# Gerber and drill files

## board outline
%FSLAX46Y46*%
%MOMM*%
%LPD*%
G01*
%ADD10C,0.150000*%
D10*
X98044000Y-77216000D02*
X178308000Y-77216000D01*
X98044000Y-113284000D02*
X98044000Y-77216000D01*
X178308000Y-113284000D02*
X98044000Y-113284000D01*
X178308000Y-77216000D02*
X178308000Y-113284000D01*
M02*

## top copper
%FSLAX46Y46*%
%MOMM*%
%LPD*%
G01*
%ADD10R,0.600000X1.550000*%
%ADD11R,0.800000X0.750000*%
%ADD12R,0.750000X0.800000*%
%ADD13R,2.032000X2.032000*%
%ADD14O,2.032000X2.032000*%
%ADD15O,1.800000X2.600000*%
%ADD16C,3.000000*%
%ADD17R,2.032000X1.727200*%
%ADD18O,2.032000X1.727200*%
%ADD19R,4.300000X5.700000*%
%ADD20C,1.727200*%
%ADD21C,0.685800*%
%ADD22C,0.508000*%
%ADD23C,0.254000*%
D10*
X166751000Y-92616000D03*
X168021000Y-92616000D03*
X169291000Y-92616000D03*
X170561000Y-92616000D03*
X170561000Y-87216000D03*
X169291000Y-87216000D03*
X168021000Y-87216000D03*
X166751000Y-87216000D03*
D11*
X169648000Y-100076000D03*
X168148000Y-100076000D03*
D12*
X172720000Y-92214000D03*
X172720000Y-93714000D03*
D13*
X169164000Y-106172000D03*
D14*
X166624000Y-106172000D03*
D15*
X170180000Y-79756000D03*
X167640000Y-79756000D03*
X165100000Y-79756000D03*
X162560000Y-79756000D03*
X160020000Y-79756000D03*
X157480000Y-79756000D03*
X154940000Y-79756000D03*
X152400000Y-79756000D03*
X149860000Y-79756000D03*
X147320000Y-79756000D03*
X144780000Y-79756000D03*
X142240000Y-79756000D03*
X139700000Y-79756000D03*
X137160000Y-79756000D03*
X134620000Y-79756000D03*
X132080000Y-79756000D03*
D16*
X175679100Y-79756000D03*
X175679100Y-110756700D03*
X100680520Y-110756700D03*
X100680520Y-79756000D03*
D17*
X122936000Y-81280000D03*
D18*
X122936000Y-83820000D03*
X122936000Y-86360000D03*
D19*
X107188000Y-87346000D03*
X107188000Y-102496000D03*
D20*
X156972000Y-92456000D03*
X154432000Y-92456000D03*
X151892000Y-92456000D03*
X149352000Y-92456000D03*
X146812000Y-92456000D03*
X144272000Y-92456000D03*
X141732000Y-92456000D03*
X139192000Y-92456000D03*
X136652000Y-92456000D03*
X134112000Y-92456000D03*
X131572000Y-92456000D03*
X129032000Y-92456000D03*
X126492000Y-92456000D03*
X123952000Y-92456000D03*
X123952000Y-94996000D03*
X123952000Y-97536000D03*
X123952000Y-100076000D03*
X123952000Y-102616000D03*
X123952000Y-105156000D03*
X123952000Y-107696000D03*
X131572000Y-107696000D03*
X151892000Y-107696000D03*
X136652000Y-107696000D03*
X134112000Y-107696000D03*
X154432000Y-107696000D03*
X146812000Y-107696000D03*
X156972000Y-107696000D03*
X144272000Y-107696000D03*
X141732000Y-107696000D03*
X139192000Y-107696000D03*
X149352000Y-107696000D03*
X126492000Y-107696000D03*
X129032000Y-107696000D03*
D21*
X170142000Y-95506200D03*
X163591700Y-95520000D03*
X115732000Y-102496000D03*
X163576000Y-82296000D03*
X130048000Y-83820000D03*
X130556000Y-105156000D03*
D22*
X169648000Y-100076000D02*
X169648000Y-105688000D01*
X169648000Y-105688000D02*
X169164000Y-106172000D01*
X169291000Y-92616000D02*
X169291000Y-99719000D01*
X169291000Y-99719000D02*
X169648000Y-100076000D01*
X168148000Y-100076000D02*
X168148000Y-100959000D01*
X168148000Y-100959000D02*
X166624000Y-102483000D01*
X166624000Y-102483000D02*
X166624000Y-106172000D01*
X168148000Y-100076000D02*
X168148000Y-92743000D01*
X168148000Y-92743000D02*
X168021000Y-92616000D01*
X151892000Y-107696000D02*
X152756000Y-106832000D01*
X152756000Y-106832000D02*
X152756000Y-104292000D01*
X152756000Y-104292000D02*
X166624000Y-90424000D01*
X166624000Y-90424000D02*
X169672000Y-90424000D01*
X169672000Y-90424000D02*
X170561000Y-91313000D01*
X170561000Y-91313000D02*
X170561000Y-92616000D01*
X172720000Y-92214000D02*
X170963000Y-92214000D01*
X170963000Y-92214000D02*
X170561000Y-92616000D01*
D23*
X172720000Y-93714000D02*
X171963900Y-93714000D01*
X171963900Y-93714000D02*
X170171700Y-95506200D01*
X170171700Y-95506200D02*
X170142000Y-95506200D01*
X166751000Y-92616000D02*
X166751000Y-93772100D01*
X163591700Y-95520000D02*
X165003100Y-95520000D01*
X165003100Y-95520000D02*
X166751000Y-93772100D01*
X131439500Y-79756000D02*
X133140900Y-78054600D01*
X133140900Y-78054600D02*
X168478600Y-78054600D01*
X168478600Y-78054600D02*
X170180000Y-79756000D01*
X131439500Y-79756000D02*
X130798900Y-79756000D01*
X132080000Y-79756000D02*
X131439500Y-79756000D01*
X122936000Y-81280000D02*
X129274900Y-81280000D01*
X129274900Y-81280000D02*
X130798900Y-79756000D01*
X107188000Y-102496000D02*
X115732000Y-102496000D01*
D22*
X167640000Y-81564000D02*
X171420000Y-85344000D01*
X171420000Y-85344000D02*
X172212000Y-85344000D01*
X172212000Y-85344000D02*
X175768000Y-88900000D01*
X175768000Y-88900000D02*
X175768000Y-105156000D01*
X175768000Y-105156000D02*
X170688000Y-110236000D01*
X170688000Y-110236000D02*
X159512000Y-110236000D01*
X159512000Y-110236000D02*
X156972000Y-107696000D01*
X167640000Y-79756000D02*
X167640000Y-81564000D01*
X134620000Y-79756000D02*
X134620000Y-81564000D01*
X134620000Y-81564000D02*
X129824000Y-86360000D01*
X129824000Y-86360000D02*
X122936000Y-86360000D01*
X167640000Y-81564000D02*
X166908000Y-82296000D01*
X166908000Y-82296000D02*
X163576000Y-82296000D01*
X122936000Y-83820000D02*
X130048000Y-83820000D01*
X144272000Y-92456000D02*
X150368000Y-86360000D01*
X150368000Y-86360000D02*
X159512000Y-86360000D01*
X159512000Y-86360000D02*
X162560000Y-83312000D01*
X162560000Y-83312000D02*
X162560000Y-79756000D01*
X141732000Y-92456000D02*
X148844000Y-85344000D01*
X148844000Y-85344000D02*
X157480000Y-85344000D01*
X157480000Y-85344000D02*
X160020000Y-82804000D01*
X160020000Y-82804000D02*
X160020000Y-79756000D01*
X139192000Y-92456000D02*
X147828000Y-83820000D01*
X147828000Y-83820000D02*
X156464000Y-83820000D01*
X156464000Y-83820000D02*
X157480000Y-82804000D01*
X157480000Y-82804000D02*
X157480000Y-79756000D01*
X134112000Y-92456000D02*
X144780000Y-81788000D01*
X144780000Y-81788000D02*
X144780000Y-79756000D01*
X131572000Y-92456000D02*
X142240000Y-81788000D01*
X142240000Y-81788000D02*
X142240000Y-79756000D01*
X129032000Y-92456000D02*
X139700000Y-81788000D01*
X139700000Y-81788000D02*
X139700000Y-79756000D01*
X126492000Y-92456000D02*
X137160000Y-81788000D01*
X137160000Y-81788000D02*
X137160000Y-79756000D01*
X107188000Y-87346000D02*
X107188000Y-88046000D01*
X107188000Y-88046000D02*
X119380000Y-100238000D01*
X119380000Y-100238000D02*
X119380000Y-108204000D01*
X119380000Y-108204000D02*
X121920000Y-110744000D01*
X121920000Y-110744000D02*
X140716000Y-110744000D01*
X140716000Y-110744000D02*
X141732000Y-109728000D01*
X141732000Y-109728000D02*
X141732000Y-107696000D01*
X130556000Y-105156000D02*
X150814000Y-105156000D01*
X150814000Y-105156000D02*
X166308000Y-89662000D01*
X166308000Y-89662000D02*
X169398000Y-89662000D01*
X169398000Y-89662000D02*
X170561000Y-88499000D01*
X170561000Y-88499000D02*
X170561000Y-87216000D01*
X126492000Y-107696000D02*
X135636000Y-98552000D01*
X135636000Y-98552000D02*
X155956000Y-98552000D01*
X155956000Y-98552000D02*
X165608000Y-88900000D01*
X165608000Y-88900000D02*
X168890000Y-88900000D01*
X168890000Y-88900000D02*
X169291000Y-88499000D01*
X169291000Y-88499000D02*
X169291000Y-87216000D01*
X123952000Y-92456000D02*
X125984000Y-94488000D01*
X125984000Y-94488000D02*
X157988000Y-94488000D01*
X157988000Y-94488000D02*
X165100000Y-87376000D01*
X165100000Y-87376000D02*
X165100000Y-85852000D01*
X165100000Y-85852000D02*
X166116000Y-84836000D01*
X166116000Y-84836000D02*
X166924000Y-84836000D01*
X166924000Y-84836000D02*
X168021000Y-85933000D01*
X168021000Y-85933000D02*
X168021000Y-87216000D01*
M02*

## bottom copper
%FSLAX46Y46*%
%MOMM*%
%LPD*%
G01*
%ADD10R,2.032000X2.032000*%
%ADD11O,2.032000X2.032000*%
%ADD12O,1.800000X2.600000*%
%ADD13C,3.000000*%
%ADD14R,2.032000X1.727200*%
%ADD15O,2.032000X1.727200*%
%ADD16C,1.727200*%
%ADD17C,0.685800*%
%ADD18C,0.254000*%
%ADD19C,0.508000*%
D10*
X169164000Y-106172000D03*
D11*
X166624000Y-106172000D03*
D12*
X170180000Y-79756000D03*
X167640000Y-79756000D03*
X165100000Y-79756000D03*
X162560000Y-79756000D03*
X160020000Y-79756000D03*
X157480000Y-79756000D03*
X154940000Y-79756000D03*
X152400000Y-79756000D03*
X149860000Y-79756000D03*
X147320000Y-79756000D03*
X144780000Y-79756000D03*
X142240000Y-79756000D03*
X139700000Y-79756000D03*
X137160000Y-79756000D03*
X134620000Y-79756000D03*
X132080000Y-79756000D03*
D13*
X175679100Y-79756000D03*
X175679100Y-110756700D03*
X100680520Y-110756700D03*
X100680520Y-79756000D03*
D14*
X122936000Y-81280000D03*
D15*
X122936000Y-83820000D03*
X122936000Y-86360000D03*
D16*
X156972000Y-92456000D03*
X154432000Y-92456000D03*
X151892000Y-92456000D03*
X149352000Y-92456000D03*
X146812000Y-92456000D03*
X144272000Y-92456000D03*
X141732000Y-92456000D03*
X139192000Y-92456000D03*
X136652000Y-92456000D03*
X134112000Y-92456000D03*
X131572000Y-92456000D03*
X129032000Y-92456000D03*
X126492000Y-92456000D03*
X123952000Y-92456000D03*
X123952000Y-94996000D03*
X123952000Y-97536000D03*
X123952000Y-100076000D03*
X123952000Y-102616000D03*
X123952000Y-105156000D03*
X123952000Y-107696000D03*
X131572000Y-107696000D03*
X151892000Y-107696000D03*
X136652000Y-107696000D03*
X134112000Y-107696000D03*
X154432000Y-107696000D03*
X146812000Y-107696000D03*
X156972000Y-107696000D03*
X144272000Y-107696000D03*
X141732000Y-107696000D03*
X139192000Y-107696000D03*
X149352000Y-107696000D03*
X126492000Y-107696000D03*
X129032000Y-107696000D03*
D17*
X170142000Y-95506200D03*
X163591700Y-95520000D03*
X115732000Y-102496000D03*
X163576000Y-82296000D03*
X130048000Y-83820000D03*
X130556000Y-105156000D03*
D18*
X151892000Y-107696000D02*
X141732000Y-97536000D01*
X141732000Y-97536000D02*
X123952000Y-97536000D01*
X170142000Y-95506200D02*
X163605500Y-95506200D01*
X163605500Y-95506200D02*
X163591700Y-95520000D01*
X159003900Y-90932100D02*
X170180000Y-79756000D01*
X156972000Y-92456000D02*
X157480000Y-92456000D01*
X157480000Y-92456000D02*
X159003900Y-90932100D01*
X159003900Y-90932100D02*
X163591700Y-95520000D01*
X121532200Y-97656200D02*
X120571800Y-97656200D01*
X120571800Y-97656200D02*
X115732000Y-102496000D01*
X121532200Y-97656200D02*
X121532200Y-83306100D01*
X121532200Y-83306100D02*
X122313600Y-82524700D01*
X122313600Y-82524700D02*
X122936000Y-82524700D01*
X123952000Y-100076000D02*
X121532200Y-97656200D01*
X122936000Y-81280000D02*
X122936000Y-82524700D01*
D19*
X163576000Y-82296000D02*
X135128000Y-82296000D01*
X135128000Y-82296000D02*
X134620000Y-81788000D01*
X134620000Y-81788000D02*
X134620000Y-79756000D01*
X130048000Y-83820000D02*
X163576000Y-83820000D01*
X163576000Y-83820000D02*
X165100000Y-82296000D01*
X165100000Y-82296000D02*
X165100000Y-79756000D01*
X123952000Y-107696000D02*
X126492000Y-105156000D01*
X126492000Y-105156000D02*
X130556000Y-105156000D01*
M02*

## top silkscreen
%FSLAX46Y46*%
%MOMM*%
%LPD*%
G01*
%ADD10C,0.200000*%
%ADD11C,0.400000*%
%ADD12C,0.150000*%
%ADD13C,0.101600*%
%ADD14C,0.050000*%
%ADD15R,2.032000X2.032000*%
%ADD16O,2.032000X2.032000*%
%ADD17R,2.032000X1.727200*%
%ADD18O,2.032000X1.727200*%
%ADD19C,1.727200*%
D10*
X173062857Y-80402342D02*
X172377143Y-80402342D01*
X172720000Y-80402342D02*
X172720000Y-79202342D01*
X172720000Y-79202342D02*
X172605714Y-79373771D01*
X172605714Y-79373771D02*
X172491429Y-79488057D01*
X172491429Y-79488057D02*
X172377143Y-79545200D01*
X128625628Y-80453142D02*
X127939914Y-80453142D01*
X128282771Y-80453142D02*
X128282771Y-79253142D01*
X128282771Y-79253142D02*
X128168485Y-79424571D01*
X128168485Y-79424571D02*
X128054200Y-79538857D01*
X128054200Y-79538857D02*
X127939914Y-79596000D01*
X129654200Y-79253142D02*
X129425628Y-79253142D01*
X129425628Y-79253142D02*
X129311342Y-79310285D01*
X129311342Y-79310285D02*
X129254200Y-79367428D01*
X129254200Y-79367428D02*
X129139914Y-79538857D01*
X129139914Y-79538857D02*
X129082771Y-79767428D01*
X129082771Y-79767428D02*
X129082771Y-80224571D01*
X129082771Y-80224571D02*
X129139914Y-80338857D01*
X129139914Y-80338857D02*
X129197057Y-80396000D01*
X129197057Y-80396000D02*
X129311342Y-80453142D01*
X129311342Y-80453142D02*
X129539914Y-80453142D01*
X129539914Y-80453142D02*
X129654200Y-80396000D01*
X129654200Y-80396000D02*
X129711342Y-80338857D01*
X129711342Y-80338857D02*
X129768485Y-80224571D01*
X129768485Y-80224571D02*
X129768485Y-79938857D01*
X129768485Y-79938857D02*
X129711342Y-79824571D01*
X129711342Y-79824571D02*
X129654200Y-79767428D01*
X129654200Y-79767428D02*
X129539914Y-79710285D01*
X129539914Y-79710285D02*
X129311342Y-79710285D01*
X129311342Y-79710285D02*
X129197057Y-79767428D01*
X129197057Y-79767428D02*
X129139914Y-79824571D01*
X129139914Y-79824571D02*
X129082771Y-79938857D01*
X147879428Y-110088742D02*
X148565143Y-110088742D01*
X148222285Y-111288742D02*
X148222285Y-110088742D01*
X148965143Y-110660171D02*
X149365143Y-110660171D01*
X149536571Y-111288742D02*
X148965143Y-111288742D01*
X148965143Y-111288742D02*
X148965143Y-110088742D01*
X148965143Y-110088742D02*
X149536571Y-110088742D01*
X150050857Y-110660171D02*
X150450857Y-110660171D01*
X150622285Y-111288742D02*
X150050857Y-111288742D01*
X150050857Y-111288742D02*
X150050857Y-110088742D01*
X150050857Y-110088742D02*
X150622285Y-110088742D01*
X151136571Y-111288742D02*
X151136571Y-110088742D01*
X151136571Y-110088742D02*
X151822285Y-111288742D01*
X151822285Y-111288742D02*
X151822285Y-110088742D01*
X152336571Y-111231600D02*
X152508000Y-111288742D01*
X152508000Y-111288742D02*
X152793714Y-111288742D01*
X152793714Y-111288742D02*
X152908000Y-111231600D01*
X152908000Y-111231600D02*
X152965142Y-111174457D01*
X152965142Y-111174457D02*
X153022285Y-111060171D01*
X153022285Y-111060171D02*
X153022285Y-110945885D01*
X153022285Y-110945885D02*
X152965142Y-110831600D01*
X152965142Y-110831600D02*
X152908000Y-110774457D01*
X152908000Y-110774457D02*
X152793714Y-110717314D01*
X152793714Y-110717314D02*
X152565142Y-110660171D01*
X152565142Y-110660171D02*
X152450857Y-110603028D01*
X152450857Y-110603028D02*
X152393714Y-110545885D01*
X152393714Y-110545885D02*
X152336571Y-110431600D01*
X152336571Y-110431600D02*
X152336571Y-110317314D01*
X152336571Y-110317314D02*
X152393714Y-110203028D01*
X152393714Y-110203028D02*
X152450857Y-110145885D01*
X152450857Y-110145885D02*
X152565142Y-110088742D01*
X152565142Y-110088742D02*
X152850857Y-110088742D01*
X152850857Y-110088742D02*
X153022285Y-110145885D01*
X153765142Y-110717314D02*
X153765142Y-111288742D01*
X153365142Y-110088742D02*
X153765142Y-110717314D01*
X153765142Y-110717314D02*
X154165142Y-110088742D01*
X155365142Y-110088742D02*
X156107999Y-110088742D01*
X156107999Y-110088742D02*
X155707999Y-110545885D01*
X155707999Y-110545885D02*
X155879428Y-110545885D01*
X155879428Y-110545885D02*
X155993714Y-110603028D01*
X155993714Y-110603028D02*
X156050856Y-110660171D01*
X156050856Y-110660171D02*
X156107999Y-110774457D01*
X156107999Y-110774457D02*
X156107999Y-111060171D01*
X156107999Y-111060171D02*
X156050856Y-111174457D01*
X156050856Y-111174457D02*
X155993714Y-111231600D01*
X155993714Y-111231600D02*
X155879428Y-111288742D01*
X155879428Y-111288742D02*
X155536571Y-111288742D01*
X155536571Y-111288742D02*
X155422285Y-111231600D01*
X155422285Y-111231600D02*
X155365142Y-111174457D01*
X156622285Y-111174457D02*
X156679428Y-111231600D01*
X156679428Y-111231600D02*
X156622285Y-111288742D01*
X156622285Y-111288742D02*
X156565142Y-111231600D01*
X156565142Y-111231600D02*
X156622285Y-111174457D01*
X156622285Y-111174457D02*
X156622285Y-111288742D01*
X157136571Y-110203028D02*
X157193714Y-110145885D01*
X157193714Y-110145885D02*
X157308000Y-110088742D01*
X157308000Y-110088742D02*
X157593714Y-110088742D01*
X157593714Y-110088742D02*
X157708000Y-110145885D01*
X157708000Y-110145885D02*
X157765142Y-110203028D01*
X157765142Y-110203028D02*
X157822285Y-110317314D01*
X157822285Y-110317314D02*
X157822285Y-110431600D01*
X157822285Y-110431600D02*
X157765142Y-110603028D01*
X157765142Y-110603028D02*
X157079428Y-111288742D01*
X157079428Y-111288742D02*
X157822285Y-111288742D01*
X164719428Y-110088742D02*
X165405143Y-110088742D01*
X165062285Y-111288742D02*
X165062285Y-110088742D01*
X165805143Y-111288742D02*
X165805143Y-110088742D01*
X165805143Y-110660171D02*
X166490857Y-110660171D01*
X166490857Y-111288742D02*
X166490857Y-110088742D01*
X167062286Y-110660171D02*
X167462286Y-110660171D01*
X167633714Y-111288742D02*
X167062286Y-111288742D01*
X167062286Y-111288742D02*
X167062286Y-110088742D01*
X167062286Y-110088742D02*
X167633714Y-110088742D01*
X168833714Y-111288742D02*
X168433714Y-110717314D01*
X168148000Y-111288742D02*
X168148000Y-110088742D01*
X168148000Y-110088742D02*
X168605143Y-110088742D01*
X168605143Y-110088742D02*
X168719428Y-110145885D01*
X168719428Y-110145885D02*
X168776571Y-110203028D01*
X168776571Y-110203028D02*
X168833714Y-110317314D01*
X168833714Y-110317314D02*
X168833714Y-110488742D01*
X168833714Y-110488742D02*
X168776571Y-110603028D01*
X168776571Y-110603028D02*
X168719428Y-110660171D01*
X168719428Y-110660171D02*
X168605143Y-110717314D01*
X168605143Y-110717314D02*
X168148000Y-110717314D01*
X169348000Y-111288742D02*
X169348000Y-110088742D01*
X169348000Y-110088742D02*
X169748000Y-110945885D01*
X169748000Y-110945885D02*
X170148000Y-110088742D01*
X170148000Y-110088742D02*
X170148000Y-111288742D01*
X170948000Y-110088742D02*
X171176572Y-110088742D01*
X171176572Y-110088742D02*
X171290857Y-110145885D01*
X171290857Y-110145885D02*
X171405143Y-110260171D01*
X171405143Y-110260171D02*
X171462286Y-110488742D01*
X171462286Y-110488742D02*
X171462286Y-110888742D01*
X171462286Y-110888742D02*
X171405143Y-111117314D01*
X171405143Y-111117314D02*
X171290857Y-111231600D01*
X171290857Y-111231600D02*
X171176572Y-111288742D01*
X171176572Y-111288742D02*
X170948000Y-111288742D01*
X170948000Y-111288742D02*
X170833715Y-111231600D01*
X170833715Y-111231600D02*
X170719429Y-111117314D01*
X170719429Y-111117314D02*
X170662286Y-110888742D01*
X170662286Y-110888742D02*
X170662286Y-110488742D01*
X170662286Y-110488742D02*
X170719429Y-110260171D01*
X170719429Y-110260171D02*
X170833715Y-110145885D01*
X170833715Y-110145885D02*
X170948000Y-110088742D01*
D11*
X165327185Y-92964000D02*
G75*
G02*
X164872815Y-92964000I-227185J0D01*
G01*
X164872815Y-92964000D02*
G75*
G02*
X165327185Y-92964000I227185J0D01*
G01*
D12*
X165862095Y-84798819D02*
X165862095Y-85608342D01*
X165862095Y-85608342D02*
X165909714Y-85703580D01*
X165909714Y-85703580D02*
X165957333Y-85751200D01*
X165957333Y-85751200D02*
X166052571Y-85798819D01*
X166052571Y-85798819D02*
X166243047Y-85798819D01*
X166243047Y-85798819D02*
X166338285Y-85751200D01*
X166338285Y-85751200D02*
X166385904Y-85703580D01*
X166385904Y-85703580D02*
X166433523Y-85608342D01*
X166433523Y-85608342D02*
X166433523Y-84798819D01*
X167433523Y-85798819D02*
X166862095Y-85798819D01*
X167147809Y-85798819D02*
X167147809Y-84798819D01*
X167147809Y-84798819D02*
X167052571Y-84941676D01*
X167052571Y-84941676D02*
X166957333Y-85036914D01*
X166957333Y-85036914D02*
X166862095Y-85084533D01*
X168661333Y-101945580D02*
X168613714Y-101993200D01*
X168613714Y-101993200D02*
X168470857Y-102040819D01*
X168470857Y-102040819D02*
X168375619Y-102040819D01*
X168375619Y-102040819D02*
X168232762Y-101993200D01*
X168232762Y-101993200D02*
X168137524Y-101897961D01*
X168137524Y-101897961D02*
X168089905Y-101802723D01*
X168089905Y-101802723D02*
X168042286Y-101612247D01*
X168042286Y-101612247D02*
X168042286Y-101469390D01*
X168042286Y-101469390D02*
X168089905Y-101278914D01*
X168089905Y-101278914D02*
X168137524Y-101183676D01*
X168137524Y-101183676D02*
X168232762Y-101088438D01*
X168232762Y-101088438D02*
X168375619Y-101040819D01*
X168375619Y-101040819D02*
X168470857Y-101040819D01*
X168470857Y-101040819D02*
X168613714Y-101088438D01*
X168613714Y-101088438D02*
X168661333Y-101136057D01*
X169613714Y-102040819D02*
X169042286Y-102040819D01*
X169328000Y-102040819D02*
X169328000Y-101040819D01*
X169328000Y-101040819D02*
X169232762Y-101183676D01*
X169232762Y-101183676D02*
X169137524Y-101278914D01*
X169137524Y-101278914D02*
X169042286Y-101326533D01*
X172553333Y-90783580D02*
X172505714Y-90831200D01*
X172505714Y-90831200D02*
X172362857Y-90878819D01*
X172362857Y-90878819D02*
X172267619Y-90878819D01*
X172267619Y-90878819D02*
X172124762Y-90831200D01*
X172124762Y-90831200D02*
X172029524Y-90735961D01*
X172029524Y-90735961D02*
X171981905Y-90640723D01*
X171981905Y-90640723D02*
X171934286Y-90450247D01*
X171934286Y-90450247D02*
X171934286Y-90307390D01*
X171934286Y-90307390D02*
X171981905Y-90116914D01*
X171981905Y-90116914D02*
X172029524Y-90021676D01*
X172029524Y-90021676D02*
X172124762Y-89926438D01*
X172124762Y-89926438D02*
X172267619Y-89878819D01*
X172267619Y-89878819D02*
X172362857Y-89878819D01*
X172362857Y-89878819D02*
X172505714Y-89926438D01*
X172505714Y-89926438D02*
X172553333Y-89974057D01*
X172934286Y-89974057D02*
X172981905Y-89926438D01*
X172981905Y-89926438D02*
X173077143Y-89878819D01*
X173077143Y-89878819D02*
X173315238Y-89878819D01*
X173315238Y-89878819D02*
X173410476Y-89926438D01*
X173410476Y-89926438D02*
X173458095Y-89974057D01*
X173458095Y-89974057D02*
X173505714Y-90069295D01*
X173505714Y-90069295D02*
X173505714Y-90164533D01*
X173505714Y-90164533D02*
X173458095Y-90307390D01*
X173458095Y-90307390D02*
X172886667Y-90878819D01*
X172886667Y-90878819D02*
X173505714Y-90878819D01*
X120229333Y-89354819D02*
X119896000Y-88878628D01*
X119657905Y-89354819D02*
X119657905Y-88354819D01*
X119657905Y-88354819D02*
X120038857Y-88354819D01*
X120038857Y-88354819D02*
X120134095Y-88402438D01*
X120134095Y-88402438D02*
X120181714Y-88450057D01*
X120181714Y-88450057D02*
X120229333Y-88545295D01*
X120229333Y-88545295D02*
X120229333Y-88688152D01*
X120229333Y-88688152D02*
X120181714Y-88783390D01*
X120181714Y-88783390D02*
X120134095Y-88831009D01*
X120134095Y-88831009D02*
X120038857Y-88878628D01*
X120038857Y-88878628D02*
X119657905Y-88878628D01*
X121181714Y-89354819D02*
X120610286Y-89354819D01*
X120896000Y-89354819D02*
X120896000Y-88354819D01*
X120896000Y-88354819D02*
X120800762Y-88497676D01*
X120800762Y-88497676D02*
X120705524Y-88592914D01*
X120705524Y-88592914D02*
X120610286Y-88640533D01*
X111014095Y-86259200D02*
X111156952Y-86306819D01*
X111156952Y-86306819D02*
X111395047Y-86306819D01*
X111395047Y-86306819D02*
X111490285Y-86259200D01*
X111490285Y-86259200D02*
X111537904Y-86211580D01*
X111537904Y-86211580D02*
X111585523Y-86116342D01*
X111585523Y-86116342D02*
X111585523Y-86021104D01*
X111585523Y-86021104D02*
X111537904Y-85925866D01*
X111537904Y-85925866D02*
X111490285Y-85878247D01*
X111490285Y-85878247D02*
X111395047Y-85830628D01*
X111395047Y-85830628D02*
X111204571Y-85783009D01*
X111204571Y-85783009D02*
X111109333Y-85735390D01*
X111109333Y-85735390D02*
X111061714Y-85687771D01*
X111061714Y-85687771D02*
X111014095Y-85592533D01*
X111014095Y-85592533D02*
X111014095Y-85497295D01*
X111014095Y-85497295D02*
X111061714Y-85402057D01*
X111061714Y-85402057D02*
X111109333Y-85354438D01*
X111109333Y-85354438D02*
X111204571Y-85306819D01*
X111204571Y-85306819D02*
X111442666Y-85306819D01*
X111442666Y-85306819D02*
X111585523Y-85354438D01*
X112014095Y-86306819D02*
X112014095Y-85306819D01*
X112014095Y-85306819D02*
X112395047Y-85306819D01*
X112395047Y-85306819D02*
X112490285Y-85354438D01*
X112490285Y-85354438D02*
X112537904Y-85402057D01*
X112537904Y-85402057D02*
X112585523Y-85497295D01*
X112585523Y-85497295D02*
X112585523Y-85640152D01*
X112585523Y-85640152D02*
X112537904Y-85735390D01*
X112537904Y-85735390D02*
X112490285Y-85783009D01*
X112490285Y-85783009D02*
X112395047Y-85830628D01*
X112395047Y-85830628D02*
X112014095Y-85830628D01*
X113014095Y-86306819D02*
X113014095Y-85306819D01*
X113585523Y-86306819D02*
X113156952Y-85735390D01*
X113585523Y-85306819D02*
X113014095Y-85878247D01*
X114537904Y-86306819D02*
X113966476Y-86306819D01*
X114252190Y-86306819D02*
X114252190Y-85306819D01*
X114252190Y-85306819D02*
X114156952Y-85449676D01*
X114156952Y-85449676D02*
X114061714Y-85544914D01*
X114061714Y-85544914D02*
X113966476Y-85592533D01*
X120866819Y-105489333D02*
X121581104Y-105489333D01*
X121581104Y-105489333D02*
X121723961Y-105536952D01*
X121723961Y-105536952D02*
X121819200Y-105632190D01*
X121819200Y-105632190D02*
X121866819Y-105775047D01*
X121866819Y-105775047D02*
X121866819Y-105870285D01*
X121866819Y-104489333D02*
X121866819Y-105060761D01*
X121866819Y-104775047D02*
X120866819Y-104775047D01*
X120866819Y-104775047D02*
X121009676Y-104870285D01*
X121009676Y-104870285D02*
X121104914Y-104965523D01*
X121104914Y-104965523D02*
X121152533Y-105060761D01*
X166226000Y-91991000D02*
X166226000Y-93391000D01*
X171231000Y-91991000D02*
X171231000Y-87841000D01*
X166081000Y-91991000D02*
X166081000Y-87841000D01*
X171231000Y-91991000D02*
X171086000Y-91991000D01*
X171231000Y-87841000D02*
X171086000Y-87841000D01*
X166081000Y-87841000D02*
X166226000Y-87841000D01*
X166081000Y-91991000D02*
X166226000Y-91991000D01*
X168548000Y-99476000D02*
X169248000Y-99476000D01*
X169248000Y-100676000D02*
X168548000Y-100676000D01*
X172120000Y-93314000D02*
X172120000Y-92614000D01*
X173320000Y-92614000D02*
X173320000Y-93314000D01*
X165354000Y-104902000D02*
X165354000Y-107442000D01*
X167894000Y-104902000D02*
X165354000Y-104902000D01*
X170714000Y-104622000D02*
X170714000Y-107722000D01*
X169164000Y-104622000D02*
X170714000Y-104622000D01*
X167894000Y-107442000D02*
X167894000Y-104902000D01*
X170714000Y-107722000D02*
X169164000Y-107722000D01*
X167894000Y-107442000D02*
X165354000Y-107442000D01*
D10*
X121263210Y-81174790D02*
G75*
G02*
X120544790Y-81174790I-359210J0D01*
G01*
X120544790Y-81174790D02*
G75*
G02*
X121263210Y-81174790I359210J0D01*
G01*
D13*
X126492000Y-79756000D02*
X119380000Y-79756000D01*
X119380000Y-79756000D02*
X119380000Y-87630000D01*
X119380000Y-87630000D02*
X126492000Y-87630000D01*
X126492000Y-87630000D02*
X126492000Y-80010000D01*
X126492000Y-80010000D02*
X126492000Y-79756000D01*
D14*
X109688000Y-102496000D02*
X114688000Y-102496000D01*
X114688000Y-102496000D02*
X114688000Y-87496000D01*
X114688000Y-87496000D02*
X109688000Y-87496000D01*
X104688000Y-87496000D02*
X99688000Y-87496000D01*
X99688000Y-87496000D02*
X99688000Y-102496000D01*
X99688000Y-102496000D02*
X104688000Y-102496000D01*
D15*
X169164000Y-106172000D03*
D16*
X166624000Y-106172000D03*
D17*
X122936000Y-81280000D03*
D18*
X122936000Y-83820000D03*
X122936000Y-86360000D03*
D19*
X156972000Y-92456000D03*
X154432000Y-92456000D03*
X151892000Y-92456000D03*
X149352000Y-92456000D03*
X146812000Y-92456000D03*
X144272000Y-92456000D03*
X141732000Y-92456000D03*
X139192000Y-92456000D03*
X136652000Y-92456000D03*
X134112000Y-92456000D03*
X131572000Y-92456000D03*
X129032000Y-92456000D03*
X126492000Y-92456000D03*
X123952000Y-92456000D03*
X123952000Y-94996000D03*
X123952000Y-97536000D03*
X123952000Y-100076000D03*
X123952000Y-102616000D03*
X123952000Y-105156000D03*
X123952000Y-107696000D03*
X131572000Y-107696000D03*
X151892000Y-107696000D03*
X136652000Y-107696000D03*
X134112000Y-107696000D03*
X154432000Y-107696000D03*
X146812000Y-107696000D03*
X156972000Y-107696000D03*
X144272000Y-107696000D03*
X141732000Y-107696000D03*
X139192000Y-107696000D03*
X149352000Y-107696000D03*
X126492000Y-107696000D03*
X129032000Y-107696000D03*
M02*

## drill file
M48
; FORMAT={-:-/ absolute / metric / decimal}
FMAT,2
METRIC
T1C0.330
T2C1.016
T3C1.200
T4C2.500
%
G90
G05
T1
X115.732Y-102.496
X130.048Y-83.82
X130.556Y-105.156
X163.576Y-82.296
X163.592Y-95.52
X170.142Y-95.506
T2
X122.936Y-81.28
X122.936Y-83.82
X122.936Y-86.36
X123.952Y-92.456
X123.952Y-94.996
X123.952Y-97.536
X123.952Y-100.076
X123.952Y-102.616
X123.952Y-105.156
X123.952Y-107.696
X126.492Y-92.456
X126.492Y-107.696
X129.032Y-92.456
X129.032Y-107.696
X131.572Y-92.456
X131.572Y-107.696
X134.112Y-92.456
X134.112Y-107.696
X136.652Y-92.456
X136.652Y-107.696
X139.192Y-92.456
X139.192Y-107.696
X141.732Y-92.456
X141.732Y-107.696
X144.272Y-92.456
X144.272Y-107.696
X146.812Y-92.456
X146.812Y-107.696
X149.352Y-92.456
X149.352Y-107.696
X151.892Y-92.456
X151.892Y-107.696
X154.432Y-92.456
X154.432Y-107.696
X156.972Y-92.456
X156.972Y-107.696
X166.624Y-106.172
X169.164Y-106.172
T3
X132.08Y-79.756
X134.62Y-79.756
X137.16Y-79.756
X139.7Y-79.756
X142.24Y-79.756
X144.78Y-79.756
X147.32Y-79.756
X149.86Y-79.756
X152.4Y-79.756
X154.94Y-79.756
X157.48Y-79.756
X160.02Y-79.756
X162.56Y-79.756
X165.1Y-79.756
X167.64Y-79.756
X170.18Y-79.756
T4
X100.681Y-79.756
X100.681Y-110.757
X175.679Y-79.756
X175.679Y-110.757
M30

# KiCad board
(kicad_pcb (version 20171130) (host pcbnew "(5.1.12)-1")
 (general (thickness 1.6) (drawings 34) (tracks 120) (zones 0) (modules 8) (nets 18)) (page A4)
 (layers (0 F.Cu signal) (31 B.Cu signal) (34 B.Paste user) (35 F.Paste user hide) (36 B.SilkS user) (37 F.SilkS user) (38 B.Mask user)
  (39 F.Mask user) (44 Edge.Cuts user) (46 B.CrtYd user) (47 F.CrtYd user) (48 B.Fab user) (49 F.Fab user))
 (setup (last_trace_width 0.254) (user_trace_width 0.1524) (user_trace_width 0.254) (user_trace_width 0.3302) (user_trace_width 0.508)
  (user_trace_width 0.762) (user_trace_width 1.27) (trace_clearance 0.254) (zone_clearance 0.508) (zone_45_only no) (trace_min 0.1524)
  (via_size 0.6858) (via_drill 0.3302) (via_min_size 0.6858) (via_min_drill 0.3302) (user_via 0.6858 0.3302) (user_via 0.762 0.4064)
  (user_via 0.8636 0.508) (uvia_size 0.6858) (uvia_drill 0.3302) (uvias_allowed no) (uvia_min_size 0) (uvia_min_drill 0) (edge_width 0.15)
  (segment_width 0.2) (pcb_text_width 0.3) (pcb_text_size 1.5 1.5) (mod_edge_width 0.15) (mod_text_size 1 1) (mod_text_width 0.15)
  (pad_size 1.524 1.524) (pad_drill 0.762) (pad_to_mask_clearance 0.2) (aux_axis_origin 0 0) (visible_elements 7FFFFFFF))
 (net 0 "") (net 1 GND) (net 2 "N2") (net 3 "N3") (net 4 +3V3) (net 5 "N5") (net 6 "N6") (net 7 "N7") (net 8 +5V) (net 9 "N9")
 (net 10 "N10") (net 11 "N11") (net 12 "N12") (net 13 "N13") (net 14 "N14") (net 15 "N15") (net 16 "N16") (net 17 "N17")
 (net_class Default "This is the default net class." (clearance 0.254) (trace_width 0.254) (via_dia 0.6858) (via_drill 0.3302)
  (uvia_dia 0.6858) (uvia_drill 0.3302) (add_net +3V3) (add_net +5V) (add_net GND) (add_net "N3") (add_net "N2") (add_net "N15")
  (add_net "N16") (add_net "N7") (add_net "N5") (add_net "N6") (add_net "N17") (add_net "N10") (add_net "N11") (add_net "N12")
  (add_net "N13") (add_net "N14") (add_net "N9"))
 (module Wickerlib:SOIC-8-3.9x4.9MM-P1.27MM (layer F.Cu) (at 168.656 89.916 90)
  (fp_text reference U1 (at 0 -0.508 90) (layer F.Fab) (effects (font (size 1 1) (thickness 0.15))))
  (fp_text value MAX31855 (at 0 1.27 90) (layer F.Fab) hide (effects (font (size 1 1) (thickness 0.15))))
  (fp_line (start -2.075 -2.43) (end -3.475 -2.43) (layer F.SilkS) (width 0.15))
  (fp_line (start -2.075 2.575) (end 2.075 2.575) (layer F.SilkS) (width 0.15))
  (fp_line (start -2.075 -2.575) (end 2.075 -2.575) (layer F.SilkS) (width 0.15))
  (fp_line (start -2.075 2.575) (end -2.075 2.43) (layer F.SilkS) (width 0.15))
  (fp_line (start 2.075 2.575) (end 2.075 2.43) (layer F.SilkS) (width 0.15))
  (fp_line (start 2.075 -2.575) (end 2.075 -2.43) (layer F.SilkS) (width 0.15))
  (fp_line (start -2.075 -2.575) (end -2.075 -2.43) (layer F.SilkS) (width 0.15))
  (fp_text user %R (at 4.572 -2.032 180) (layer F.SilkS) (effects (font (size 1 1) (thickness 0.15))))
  (pad 1 smd rect (at -2.7 -1.905 90) (size 1.55 0.6) (layers F.Cu F.Paste F.Mask) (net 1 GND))
  (pad 2 smd rect (at -2.7 -0.635 90) (size 1.55 0.6) (layers F.Cu F.Paste F.Mask) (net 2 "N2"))
  (pad 3 smd rect (at -2.7 0.635 90) (size 1.55 0.6) (layers F.Cu F.Paste F.Mask) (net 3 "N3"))
  (pad 4 smd rect (at -2.7 1.905 90) (size 1.55 0.6) (layers F.Cu F.Paste F.Mask) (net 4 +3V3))
  (pad 5 smd rect (at 2.7 1.905 90) (size 1.55 0.6) (layers F.Cu F.Paste F.Mask) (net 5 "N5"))
  (pad 6 smd rect (at 2.7 0.635 90) (size 1.55 0.6) (layers F.Cu F.Paste F.Mask) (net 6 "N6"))
  (pad 7 smd rect (at 2.7 -0.635 90) (size 1.55 0.6) (layers F.Cu F.Paste F.Mask) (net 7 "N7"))
  (pad 8 smd rect (at 2.7 -1.905 90) (size 1.55 0.6) (layers F.Cu F.Paste F.Mask)))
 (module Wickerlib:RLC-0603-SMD (layer F.Cu) (at 168.898 100.076 180)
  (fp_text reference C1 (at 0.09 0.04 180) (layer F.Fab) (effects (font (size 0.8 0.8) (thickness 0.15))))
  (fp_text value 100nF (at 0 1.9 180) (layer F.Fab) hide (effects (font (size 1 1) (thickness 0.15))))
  (fp_line (start 0.35 0.6) (end -0.35 0.6) (layer F.SilkS) (width 0.15))
  (fp_line (start -0.35 -0.6) (end 0.35 -0.6) (layer F.SilkS) (width 0.15))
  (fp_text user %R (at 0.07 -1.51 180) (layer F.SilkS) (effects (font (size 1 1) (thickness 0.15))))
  (pad 1 smd rect (at -0.75 0 180) (size 0.8 0.75) (layers F.Cu F.Paste F.Mask) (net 3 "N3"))
  (pad 2 smd rect (at 0.75 0 180) (size 0.8 0.75) (layers F.Cu F.Paste F.Mask) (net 2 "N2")))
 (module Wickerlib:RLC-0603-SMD (layer F.Cu) (at 172.72 92.964 270)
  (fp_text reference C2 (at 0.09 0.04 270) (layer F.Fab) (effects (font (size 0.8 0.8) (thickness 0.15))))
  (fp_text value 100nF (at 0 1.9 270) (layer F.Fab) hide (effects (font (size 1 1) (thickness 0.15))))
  (fp_line (start 0.35 0.6) (end -0.35 0.6) (layer F.SilkS) (width 0.15))
  (fp_line (start -0.35 -0.6) (end 0.35 -0.6) (layer F.SilkS) (width 0.15))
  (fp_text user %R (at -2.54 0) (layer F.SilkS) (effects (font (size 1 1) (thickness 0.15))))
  (pad 1 smd rect (at -0.75 0 270) (size 0.8 0.75) (layers F.Cu F.Paste F.Mask) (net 4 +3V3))
  (pad 2 smd rect (at 0.75 0 270) (size 0.8 0.75) (layers F.Cu F.Paste F.Mask) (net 1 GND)))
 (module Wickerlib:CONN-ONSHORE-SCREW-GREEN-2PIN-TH (layer F.Cu) (at 169.164 106.172 270)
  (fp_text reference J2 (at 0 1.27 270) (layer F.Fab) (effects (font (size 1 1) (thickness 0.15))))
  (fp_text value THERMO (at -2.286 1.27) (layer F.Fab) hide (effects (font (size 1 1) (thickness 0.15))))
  (fp_line (start -1.27 3.81) (end 1.27 3.81) (layer F.SilkS) (width 0.15))
  (fp_line (start -1.27 1.27) (end -1.27 3.81) (layer F.SilkS) (width 0.15))
  (fp_line (start -1.55 -1.55) (end 1.55 -1.55) (layer F.SilkS) (width 0.15))
  (fp_line (start -1.55 0) (end -1.55 -1.55) (layer F.SilkS) (width 0.15))
  (fp_line (start 1.27 1.27) (end -1.27 1.27) (layer F.SilkS) (width 0.15))
  (fp_line (start 1.55 -1.55) (end 1.55 0) (layer F.SilkS) (width 0.15))
  (fp_line (start 1.27 1.27) (end 1.27 3.81) (layer F.SilkS) (width 0.15))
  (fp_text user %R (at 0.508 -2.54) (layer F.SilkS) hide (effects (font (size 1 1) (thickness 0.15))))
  (pad 1 thru_hole rect (at 0 0 270) (size 2.032 2.032) (drill 1.016) (layers *.Cu *.Mask F.SilkS) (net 3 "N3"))
  (pad 2 thru_hole oval (at 0 2.54 270) (size 2.032 2.032) (drill 1.016) (layers *.Cu *.Mask F.SilkS) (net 2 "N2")))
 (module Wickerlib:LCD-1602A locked (layer B.Cu) (at 170.18 79.756 180)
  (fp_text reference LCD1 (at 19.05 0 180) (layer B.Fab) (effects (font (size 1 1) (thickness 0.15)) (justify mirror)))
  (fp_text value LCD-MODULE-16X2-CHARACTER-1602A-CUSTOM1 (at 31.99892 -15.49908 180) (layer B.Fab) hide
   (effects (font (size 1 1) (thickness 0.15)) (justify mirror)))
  (pad 1 thru_hole oval (at 0 0 180) (size 1.8 2.6) (drill 1.2) (layers *.Cu *.Mask B.SilkS) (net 1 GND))
  (pad 2 thru_hole oval (at 2.54 0 180) (size 1.8 2.6) (drill 1.2) (layers *.Cu *.Mask B.SilkS) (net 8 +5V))
  (pad 3 thru_hole oval (at 5.08 0 180) (size 1.8 2.6) (drill 1.2) (layers *.Cu *.Mask B.SilkS) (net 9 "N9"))
  (pad 4 thru_hole oval (at 7.62 0 180) (size 1.8 2.6) (drill 1.2) (layers *.Cu *.Mask B.SilkS) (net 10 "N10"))
  (pad 5 thru_hole oval (at 10.16 0 180) (size 1.8 2.6) (drill 1.2) (layers *.Cu *.Mask B.SilkS) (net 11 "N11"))
  (pad 6 thru_hole oval (at 12.7 0 180) (size 1.8 2.6) (drill 1.2) (layers *.Cu *.Mask B.SilkS) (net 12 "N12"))
  (pad 7 thru_hole oval (at 15.24 0 180) (size 1.8 2.6) (drill 1.2) (layers *.Cu *.Mask B.SilkS))
  (pad 8 thru_hole oval (at 17.78 0 180) (size 1.8 2.6) (drill 1.2) (layers *.Cu *.Mask B.SilkS))
  (pad 9 thru_hole oval (at 20.32 0 180) (size 1.8 2.6) (drill 1.2) (layers *.Cu *.Mask B.SilkS))
  (pad 10 thru_hole oval (at 22.86 0 180) (size 1.8 2.6) (drill 1.2) (layers *.Cu *.Mask B.SilkS))
  (pad 11 thru_hole oval (at 25.4 0 180) (size 1.8 2.6) (drill 1.2) (layers *.Cu *.Mask B.SilkS) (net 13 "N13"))
  (pad 12 thru_hole oval (at 27.94 0 180) (size 1.8 2.6) (drill 1.2) (layers *.Cu *.Mask B.SilkS) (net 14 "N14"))
  (pad 13 thru_hole oval (at 30.48 0 180) (size 1.8 2.6) (drill 1.2) (layers *.Cu *.Mask B.SilkS) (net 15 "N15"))
  (pad 14 thru_hole oval (at 33.02 0 180) (size 1.8 2.6) (drill 1.2) (layers *.Cu *.Mask B.SilkS) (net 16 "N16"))
  (pad 15 thru_hole oval (at 35.56 0 180) (size 1.8 2.6) (drill 1.2) (layers *.Cu *.Mask B.SilkS) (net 8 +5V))
  (pad 16 thru_hole oval (at 38.1 0 180) (size 1.8 2.6) (drill 1.2) (layers *.Cu *.Mask B.SilkS) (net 1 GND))
  (pad 0 thru_hole circle (at -5.4991 0 180) (size 3 3) (drill 2.5) (layers *.Cu *.Mask B.SilkS))
  (pad 0 thru_hole circle (at -5.4991 -31.0007 180) (size 3 3) (drill 2.5) (layers *.Cu *.Mask B.SilkS))
  (pad 0 thru_hole circle (at 69.49948 -31.0007 180) (size 3 3) (drill 2.5) (layers *.Cu *.Mask B.SilkS))
  (pad 0 thru_hole circle (at 69.49948 0 180) (size 3 3) (drill 2.5) (layers *.Cu *.Mask B.SilkS)))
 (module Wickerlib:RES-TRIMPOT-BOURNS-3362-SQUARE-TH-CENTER (layer F.Cu) (at 122.936 83.82)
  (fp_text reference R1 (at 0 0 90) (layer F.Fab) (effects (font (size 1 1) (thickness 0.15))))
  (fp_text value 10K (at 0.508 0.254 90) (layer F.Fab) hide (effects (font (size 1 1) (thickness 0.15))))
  (fp_circle (center -2.032 -2.64521) (end -1.778 -2.39121) (layer F.SilkS) (width 0.2))
  (fp_line (start 3.556 -4.064) (end -3.556 -4.064) (layer F.SilkS) (width 0.1016))
  (fp_line (start -3.556 -4.064) (end -3.556 3.81) (layer F.SilkS) (width 0.1016))
  (fp_line (start -3.556 3.81) (end 3.556 3.81) (layer F.SilkS) (width 0.1016))
  (fp_line (start 3.556 3.81) (end 3.556 -3.81) (layer F.SilkS) (width 0.1016))
  (fp_line (start 3.556 -3.81) (end 3.556 -4.064) (layer F.SilkS) (width 0.1016))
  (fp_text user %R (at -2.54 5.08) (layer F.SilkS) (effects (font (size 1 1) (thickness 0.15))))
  (pad 1 thru_hole rect (at 0 -2.54) (size 2.032 1.7272) (drill 1.016) (layers *.Cu *.Mask F.SilkS) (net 1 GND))
  (pad 2 thru_hole oval (at 0 0) (size 2.032 1.7272) (drill 1.016) (layers *.Cu *.Mask F.SilkS) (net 9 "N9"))
  (pad 3 thru_hole oval (at 0 2.54) (size 2.032 1.7272) (drill 1.016) (layers *.Cu *.Mask F.SilkS) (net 8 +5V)))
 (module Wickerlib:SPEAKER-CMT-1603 (layer F.Cu) (at 107.188 94.996 270)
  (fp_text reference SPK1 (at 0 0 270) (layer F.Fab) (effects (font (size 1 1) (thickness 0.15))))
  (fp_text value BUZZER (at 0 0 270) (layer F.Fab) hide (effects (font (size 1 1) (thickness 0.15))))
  (fp_line (start 7.5 -2.5) (end 7.5 -7.5) (layer F.SilkS) (width 0.05))
  (fp_line (start 7.5 -7.5) (end -7.5 -7.5) (layer F.SilkS) (width 0.05))
  (fp_line (start -7.5 -7.5) (end -7.5 -2.5) (layer F.SilkS) (width 0.05))
  (fp_line (start -7.5 2.5) (end -7.5 7.5) (layer F.SilkS) (width 0.05))
  (fp_line (start -7.5 7.5) (end 7.5 7.5) (layer F.SilkS) (width 0.05))
  (fp_line (start 7.5 7.5) (end 7.5 2.5) (layer F.SilkS) (width 0.05))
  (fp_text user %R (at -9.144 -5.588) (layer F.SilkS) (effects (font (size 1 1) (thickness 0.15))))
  (pad 1 smd rect (at -7.65 0 270) (size 5.7 4.3) (layers F.Cu F.Paste F.Mask) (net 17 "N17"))
  (pad 2 smd rect (at 7.5 0 270) (size 5.7 4.3) (layers F.Cu F.Paste F.Mask) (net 1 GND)))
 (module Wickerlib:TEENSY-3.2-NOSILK (layer F.Cu) (at 146.812 102.616 270)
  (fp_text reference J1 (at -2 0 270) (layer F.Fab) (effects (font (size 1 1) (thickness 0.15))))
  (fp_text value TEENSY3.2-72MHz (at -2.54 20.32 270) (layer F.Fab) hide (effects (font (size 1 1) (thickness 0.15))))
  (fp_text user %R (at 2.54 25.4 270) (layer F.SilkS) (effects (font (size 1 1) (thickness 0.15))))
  (pad G1 thru_hole circle (at -10.16 -10.16 270) (size 1.7272 1.7272) (drill 1.016) (layers *.Cu *.Mask F.SilkS) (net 1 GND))
  (pad 0 thru_hole circle (at -10.16 -7.62 270) (size 1.7272 1.7272) (drill 1.016) (layers *.Cu *.Mask F.SilkS))
  (pad 1 thru_hole circle (at -10.16 -5.08 270) (size 1.7272 1.7272) (drill 1.016) (layers *.Cu *.Mask F.SilkS))
  (pad 2 thru_hole circle (at -10.16 -2.54 270) (size 1.7272 1.7272) (drill 1.016) (layers *.Cu *.Mask F.SilkS))
  (pad 3 thru_hole circle (at -10.16 0 270) (size 1.7272 1.7272) (drill 1.016) (layers *.Cu *.Mask F.SilkS))
  (pad 4 thru_hole circle (at -10.16 2.54 270) (size 1.7272 1.7272) (drill 1.016) (layers *.Cu *.Mask F.SilkS) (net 10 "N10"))
  (pad 5 thru_hole circle (at -10.16 5.08 270) (size 1.7272 1.7272) (drill 1.016) (layers *.Cu *.Mask F.SilkS) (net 11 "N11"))
  (pad 6 thru_hole circle (at -10.16 7.62 270) (size 1.7272 1.7272) (drill 1.016) (layers *.Cu *.Mask F.SilkS) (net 12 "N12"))
  (pad 7 thru_hole circle (at -10.16 10.16 270) (size 1.7272 1.7272) (drill 1.016) (layers *.Cu *.Mask F.SilkS))
  (pad 8 thru_hole circle (at -10.16 12.7 270) (size 1.7272 1.7272) (drill 1.016) (layers *.Cu *.Mask F.SilkS) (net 13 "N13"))
  (pad 9 thru_hole circle (at -10.16 15.24 270) (size 1.7272 1.7272) (drill 1.016) (layers *.Cu *.Mask F.SilkS) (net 14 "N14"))
  (pad 10 thru_hole circle (at -10.16 17.78 270) (size 1.7272 1.7272) (drill 1.016) (layers *.Cu *.Mask F.SilkS) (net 15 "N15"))
  (pad 11 thru_hole circle (at -10.16 20.32 270) (size 1.7272 1.7272) (drill 1.016) (layers *.Cu *.Mask F.SilkS) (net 16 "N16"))
  (pad 12 thru_hole circle (at -10.16 22.86 270) (size 1.7272 1.7272) (drill 1.016) (layers *.Cu *.Mask F.SilkS) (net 7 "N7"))
  (pad VBAT thru_hole circle (at -7.62 22.86 270) (size 1.7272 1.7272) (drill 1.016) (layers *.Cu *.Mask F.SilkS))
  (pad 3V1 thru_hole circle (at -5.08 22.86 270) (size 1.7272 1.7272) (drill 1.016) (layers *.Cu *.Mask F.SilkS) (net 4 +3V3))
  (pad G2 thru_hole circle (at -2.54 22.86 270) (size 1.7272 1.7272) (drill 1.016) (layers *.Cu *.Mask F.SilkS) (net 1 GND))
  (pad PGM thru_hole circle (at 0 22.86 270) (size 1.7272 1.7272) (drill 1.016) (layers *.Cu *.Mask F.SilkS))
  (pad DAC thru_hole circle (at 2.54 22.86 270) (size 1.7272 1.7272) (drill 1.016) (layers *.Cu *.Mask F.SilkS))
  (pad 13 thru_hole circle (at 5.08 22.86 270) (size 1.7272 1.7272) (drill 1.016) (layers *.Cu *.Mask F.SilkS) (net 5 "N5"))
  (pad 16 thru_hole circle (at 5.08 15.24 270) (size 1.7272 1.7272) (drill 1.016) (layers *.Cu *.Mask F.SilkS))
  (pad 3V2 thru_hole circle (at 5.08 -5.08 270) (size 1.7272 1.7272) (drill 1.016) (layers *.Cu *.Mask F.SilkS) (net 4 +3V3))
  (pad 18 thru_hole circle (at 5.08 10.16 270) (size 1.7272 1.7272) (drill 1.016) (layers *.Cu *.Mask F.SilkS))
  (pad 17 thru_hole circle (at 5.08 12.7 270) (size 1.7272 1.7272) (drill 1.016) (layers *.Cu *.Mask F.SilkS))
  (pad AG thru_hole circle (at 5.08 -7.62 270) (size 1.7272 1.7272) (drill 1.016) (layers *.Cu *.Mask F.SilkS))
  (pad 22 thru_hole circle (at 5.08 0 270) (size 1.7272 1.7272) (drill 1.016) (layers *.Cu *.Mask F.SilkS))
  (pad VIN thru_hole circle (at 5.08 -10.16 270) (size 1.7272 1.7272) (drill 1.016) (layers *.Cu *.Mask F.SilkS) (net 8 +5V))
  (pad 21 thru_hole circle (at 5.08 2.54 270) (size 1.7272 1.7272) (drill 1.016) (layers *.Cu *.Mask F.SilkS))
  (pad 20 thru_hole circle (at 5.08 5.08 270) (size 1.7272 1.7272) (drill 1.016) (layers *.Cu *.Mask F.SilkS) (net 17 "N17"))
  (pad 19 thru_hole circle (at 5.08 7.62 270) (size 1.7272 1.7272) (drill 1.016) (layers *.Cu *.Mask F.SilkS))
  (pad 23 thru_hole circle (at 5.08 -2.54 270) (size 1.7272 1.7272) (drill 1.016) (layers *.Cu *.Mask F.SilkS))
  (pad 14 thru_hole circle (at 5.08 20.32 270) (size 1.7272 1.7272) (drill 1.016) (layers *.Cu *.Mask F.SilkS) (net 6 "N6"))
  (pad 15 thru_hole circle (at 5.08 17.78 270) (size 1.7272 1.7272) (drill 1.016) (layers *.Cu *.Mask F.SilkS)))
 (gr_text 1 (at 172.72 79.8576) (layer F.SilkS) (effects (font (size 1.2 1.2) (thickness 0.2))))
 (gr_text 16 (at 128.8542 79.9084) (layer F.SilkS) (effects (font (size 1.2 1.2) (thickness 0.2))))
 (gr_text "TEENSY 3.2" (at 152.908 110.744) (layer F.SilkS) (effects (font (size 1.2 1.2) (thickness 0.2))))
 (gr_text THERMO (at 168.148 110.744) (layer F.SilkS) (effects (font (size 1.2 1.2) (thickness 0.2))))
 (gr_line (start 98.044 77.216) (end 178.308 77.216) (layer Edge.Cuts) (width 0.15))
 (gr_line (start 98.044 113.284) (end 98.044 77.216) (layer Edge.Cuts) (width 0.15))
 (gr_line (start 178.308 113.284) (end 98.044 113.284) (layer Edge.Cuts) (width 0.15))
 (gr_line (start 178.308 77.216) (end 178.308 113.284) (layer Edge.Cuts) (width 0.15))
 (gr_circle (center 165.1 92.964) (end 165.3032 93.0656) (layer F.SilkS) (width 0.4))
 (segment (start 169.648 100.076) (end 169.648 105.688) (width 0.508) (layer F.Cu) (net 3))
 (segment (start 169.648 105.688) (end 169.164 106.172) (width 0.508) (layer F.Cu) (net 3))
 (segment (start 169.291 92.616) (end 169.291 99.719) (width 0.508) (layer F.Cu) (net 3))
 (segment (start 169.291 99.719) (end 169.648 100.076) (width 0.508) (layer F.Cu) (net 3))
 (segment (start 168.148 100.076) (end 168.148 100.959) (width 0.508) (layer F.Cu) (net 2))
 (segment (start 168.148 100.959) (end 166.624 102.483) (width 0.508) (layer F.Cu) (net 2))
 (segment (start 166.624 102.483) (end 166.624 106.172) (width 0.508) (layer F.Cu) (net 2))
 (segment (start 168.148 100.076) (end 168.148 92.743) (width 0.508) (layer F.Cu) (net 2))
 (segment (start 168.148 92.743) (end 168.021 92.616) (width 0.508) (layer F.Cu) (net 2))
 (segment (start 151.892 107.696) (end 141.732 97.536) (width 0.254) (layer B.Cu) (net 4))
 (segment (start 141.732 97.536) (end 123.952 97.536) (width 0.254) (layer B.Cu) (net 4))
 (segment (start 151.892 107.696) (end 152.756 106.832) (width 0.508) (layer F.Cu) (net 4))
 (segment (start 152.756 106.832) (end 152.756 104.292) (width 0.508) (layer F.Cu) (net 4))
 (segment (start 152.756 104.292) (end 166.624 90.424) (width 0.508) (layer F.Cu) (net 4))
 (segment (start 166.624 90.424) (end 169.672 90.424) (width 0.508) (layer F.Cu) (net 4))
 (segment (start 169.672 90.424) (end 170.561 91.313) (width 0.508) (layer F.Cu) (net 4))
 (segment (start 170.561 91.313) (end 170.561 92.616) (width 0.508) (layer F.Cu) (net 4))
 (segment (start 172.72 92.214) (end 170.963 92.214) (width 0.508) (layer F.Cu) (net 4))
 (segment (start 170.963 92.214) (end 170.561 92.616) (width 0.508) (layer F.Cu) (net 4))
 (segment (start 172.72 93.714) (end 171.9639 93.714) (width 0.254) (layer F.Cu) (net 1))
 (segment (start 171.9639 93.714) (end 170.1717 95.5062) (width 0.254) (layer F.Cu) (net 1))
 (segment (start 170.1717 95.5062) (end 170.142 95.5062) (width 0.254) (layer F.Cu) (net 1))
 (segment (start 170.142 95.5062) (end 163.6055 95.5062) (width 0.254) (layer B.Cu) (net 1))
 (segment (start 163.6055 95.5062) (end 163.5917 95.52) (width 0.254) (layer B.Cu) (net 1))
 (segment (start 159.0039 90.9321) (end 170.18 79.756) (width 0.254) (layer B.Cu) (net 1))
 (segment (start 156.972 92.456) (end 157.48 92.456) (width 0.254) (layer B.Cu) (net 1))
 (segment (start 157.48 92.456) (end 159.0039 90.9321) (width 0.254) (layer B.Cu) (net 1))
 (segment (start 159.0039 90.9321) (end 163.5917 95.52) (width 0.254) (layer B.Cu) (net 1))
 (segment (start 166.751 92.616) (end 166.751 93.7721) (width 0.254) (layer F.Cu) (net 1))
 (segment (start 163.5917 95.52) (end 165.0031 95.52) (width 0.254) (layer F.Cu) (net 1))
 (segment (start 165.0031 95.52) (end 166.751 93.7721) (width 0.254) (layer F.Cu) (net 1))
 (segment (start 131.4395 79.756) (end 133.1409 78.0546) (width 0.254) (layer F.Cu) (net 1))
 (segment (start 133.1409 78.0546) (end 168.4786 78.0546) (width 0.254) (layer F.Cu) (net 1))
 (segment (start 168.4786 78.0546) (end 170.18 79.756) (width 0.254) (layer F.Cu) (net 1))
 (segment (start 131.4395 79.756) (end 130.7989 79.756) (width 0.254) (layer F.Cu) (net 1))
 (segment (start 132.08 79.756) (end 131.4395 79.756) (width 0.254) (layer F.Cu) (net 1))
 (segment (start 122.936 81.28) (end 129.2749 81.28) (width 0.254) (layer F.Cu) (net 1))
 (segment (start 129.2749 81.28) (end 130.7989 79.756) (width 0.254) (layer F.Cu) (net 1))
 (segment (start 107.188 102.496) (end 115.732 102.496) (width 0.254) (layer F.Cu) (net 1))
 (segment (start 121.5322 97.6562) (end 120.5718 97.6562) (width 0.254) (layer B.Cu) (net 1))
 (segment (start 120.5718 97.6562) (end 115.732 102.496) (width 0.254) (layer B.Cu) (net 1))
 (segment (start 121.5322 97.6562) (end 121.5322 83.3061) (width 0.254) (layer B.Cu) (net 1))
 (segment (start 121.5322 83.3061) (end 122.3136 82.5247) (width 0.254) (layer B.Cu) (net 1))
 (segment (start 122.3136 82.5247) (end 122.936 82.5247) (width 0.254) (layer B.Cu) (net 1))
 (segment (start 123.952 100.076) (end 121.5322 97.6562) (width 0.254) (layer B.Cu) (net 1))
 (segment (start 122.936 81.28) (end 122.936 82.5247) (width 0.254) (layer B.Cu) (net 1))
 (via (at 170.142 95.5062) (size 0.6858) (layers F.Cu B.Cu) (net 1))
 (via (at 163.5917 95.52) (size 0.6858) (layers F.Cu B.Cu) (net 1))
 (via (at 115.732 102.496) (size 0.6858) (layers F.Cu B.Cu) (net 1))
 (segment (start 167.64 81.564) (end 171.42 85.344) (width 0.508) (layer F.Cu) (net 8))
 (segment (start 171.42 85.344) (end 172.212 85.344) (width 0.508) (layer F.Cu) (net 8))
 (segment (start 172.212 85.344) (end 175.768 88.9) (width 0.508) (layer F.Cu) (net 8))
 (segment (start 175.768 88.9) (end 175.768 105.156) (width 0.508) (layer F.Cu) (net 8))
 (segment (start 175.768 105.156) (end 170.688 110.236) (width 0.508) (layer F.Cu) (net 8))
 (segment (start 170.688 110.236) (end 159.512 110.236) (width 0.508) (layer F.Cu) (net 8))
 (segment (start 159.512 110.236) (end 156.972 107.696) (width 0.508) (layer F.Cu) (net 8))
 (segment (start 167.64 79.756) (end 167.64 81.564) (width 0.508) (layer F.Cu) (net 8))
 (segment (start 134.62 79.756) (end 134.62 81.564) (width 0.508) (layer F.Cu) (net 8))
 (segment (start 134.62 81.564) (end 129.824 86.36) (width 0.508) (layer F.Cu) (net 8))
 (segment (start 129.824 86.36) (end 122.936 86.36) (width 0.508) (layer F.Cu) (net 8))
 (segment (start 167.64 81.564) (end 166.908 82.296) (width 0.508) (layer F.Cu) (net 8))
 (segment (start 166.908 82.296) (end 163.576 82.296) (width 0.508) (layer F.Cu) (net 8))
 (segment (start 163.576 82.296) (end 135.128 82.296) (width 0.508) (layer B.Cu) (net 8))
 (segment (start 135.128 82.296) (end 134.62 81.788) (width 0.508) (layer B.Cu) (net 8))
 (segment (start 134.62 81.788) (end 134.62 79.756) (width 0.508) (layer B.Cu) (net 8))
 (via (at 163.576 82.296) (size 0.6858) (layers F.Cu B.Cu) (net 8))
 (segment (start 122.936 83.82) (end 130.048 83.82) (width 0.508) (layer F.Cu) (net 9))
 (segment (start 130.048 83.82) (end 163.576 83.82) (width 0.508) (layer B.Cu) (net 9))
 (segment (start 163.576 83.82) (end 165.1 82.296) (width 0.508) (layer B.Cu) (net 9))
 (segment (start 165.1 82.296) (end 165.1 79.756) (width 0.508) (layer B.Cu) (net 9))
 (via (at 130.048 83.82) (size 0.6858) (layers F.Cu B.Cu) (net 9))
 (segment (start 144.272 92.456) (end 150.368 86.36) (width 0.508) (layer F.Cu) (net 10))
 (segment (start 150.368 86.36) (end 159.512 86.36) (width 0.508) (layer F.Cu) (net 10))
 (segment (start 159.512 86.36) (end 162.56 83.312) (width 0.508) (layer F.Cu) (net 10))
 (segment (start 162.56 83.312) (end 162.56 79.756) (width 0.508) (layer F.Cu) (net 10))
 (segment (start 141.732 92.456) (end 148.844 85.344) (width 0.508) (layer F.Cu) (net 11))
 (segment (start 148.844 85.344) (end 157.48 85.344) (width 0.508) (layer F.Cu) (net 11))
 (segment (start 157.48 85.344) (end 160.02 82.804) (width 0.508) (layer F.Cu) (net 11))
 (segment (start 160.02 82.804) (end 160.02 79.756) (width 0.508) (layer F.Cu) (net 11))
 (segment (start 139.192 92.456) (end 147.828 83.82) (width 0.508) (layer F.Cu) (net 12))
 (segment (start 147.828 83.82) (end 156.464 83.82) (width 0.508) (layer F.Cu) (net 12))
 (segment (start 156.464 83.82) (end 157.48 82.804) (width 0.508) (layer F.Cu) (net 12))
 (segment (start 157.48 82.804) (end 157.48 79.756) (width 0.508) (layer F.Cu) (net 12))
 (segment (start 134.112 92.456) (end 144.78 81.788) (width 0.508) (layer F.Cu) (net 13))
 (segment (start 144.78 81.788) (end 144.78 79.756) (width 0.508) (layer F.Cu) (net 13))
 (segment (start 131.572 92.456) (end 142.24 81.788) (width 0.508) (layer F.Cu) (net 14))
 (segment (start 142.24 81.788) (end 142.24 79.756) (width 0.508) (layer F.Cu) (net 14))
 (segment (start 129.032 92.456) (end 139.7 81.788) (width 0.508) (layer F.Cu) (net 15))
 (segment (start 139.7 81.788) (end 139.7 79.756) (width 0.508) (layer F.Cu) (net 15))
 (segment (start 126.492 92.456) (end 137.16 81.788) (width 0.508) (layer F.Cu) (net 16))
 (segment (start 137.16 81.788) (end 137.16 79.756) (width 0.508) (layer F.Cu) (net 16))
 (segment (start 107.188 87.346) (end 107.188 88.046) (width 0.508) (layer F.Cu) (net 17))
 (segment (start 107.188 88.046) (end 119.38 100.238) (width 0.508) (layer F.Cu) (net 17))
 (segment (start 119.38 100.238) (end 119.38 108.204) (width 0.508) (layer F.Cu) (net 17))
 (segment (start 119.38 108.204) (end 121.92 110.744) (width 0.508) (layer F.Cu) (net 17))
 (segment (start 121.92 110.744) (end 140.716 110.744) (width 0.508) (layer F.Cu) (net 17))
 (segment (start 140.716 110.744) (end 141.732 109.728) (width 0.508) (layer F.Cu) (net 17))
 (segment (start 141.732 109.728) (end 141.732 107.696) (width 0.508) (layer F.Cu) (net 17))
 (segment (start 123.952 107.696) (end 126.492 105.156) (width 0.508) (layer B.Cu) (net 5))
 (segment (start 126.492 105.156) (end 130.556 105.156) (width 0.508) (layer B.Cu) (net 5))
 (segment (start 130.556 105.156) (end 150.814 105.156) (width 0.508) (layer F.Cu) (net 5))
 (segment (start 150.814 105.156) (end 166.308 89.662) (width 0.508) (layer F.Cu) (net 5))
 (segment (start 166.308 89.662) (end 169.398 89.662) (width 0.508) (layer F.Cu) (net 5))
 (segment (start 169.398 89.662) (end 170.561 88.499) (width 0.508) (layer F.Cu) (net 5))
 (segment (start 170.561 88.499) (end 170.561 87.216) (width 0.508) (layer F.Cu) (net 5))
 (via (at 130.556 105.156) (size 0.6858) (layers F.Cu B.Cu) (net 5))
 (segment (start 126.492 107.696) (end 135.636 98.552) (width 0.508) (layer F.Cu) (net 6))
 (segment (start 135.636 98.552) (end 155.956 98.552) (width 0.508) (layer F.Cu) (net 6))
 (segment (start 155.956 98.552) (end 165.608 88.9) (width 0.508) (layer F.Cu) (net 6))
 (segment (start 165.608 88.9) (end 168.89 88.9) (width 0.508) (layer F.Cu) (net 6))
 (segment (start 168.89 88.9) (end 169.291 88.499) (width 0.508) (layer F.Cu) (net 6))
 (segment (start 169.291 88.499) (end 169.291 87.216) (width 0.508) (layer F.Cu) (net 6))
 (segment (start 123.952 92.456) (end 125.984 94.488) (width 0.508) (layer F.Cu) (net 7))
 (segment (start 125.984 94.488) (end 157.988 94.488) (width 0.508) (layer F.Cu) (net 7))
 (segment (start 157.988 94.488) (end 165.1 87.376) (width 0.508) (layer F.Cu) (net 7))
 (segment (start 165.1 87.376) (end 165.1 85.852) (width 0.508) (layer F.Cu) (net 7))
 (segment (start 165.1 85.852) (end 166.116 84.836) (width 0.508) (layer F.Cu) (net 7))
 (segment (start 166.116 84.836) (end 166.924 84.836) (width 0.508) (layer F.Cu) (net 7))
 (segment (start 166.924 84.836) (end 168.021 85.933) (width 0.508) (layer F.Cu) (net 7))
 (segment (start 168.021 85.933) (end 168.021 87.216) (width 0.508) (layer F.Cu) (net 7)))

